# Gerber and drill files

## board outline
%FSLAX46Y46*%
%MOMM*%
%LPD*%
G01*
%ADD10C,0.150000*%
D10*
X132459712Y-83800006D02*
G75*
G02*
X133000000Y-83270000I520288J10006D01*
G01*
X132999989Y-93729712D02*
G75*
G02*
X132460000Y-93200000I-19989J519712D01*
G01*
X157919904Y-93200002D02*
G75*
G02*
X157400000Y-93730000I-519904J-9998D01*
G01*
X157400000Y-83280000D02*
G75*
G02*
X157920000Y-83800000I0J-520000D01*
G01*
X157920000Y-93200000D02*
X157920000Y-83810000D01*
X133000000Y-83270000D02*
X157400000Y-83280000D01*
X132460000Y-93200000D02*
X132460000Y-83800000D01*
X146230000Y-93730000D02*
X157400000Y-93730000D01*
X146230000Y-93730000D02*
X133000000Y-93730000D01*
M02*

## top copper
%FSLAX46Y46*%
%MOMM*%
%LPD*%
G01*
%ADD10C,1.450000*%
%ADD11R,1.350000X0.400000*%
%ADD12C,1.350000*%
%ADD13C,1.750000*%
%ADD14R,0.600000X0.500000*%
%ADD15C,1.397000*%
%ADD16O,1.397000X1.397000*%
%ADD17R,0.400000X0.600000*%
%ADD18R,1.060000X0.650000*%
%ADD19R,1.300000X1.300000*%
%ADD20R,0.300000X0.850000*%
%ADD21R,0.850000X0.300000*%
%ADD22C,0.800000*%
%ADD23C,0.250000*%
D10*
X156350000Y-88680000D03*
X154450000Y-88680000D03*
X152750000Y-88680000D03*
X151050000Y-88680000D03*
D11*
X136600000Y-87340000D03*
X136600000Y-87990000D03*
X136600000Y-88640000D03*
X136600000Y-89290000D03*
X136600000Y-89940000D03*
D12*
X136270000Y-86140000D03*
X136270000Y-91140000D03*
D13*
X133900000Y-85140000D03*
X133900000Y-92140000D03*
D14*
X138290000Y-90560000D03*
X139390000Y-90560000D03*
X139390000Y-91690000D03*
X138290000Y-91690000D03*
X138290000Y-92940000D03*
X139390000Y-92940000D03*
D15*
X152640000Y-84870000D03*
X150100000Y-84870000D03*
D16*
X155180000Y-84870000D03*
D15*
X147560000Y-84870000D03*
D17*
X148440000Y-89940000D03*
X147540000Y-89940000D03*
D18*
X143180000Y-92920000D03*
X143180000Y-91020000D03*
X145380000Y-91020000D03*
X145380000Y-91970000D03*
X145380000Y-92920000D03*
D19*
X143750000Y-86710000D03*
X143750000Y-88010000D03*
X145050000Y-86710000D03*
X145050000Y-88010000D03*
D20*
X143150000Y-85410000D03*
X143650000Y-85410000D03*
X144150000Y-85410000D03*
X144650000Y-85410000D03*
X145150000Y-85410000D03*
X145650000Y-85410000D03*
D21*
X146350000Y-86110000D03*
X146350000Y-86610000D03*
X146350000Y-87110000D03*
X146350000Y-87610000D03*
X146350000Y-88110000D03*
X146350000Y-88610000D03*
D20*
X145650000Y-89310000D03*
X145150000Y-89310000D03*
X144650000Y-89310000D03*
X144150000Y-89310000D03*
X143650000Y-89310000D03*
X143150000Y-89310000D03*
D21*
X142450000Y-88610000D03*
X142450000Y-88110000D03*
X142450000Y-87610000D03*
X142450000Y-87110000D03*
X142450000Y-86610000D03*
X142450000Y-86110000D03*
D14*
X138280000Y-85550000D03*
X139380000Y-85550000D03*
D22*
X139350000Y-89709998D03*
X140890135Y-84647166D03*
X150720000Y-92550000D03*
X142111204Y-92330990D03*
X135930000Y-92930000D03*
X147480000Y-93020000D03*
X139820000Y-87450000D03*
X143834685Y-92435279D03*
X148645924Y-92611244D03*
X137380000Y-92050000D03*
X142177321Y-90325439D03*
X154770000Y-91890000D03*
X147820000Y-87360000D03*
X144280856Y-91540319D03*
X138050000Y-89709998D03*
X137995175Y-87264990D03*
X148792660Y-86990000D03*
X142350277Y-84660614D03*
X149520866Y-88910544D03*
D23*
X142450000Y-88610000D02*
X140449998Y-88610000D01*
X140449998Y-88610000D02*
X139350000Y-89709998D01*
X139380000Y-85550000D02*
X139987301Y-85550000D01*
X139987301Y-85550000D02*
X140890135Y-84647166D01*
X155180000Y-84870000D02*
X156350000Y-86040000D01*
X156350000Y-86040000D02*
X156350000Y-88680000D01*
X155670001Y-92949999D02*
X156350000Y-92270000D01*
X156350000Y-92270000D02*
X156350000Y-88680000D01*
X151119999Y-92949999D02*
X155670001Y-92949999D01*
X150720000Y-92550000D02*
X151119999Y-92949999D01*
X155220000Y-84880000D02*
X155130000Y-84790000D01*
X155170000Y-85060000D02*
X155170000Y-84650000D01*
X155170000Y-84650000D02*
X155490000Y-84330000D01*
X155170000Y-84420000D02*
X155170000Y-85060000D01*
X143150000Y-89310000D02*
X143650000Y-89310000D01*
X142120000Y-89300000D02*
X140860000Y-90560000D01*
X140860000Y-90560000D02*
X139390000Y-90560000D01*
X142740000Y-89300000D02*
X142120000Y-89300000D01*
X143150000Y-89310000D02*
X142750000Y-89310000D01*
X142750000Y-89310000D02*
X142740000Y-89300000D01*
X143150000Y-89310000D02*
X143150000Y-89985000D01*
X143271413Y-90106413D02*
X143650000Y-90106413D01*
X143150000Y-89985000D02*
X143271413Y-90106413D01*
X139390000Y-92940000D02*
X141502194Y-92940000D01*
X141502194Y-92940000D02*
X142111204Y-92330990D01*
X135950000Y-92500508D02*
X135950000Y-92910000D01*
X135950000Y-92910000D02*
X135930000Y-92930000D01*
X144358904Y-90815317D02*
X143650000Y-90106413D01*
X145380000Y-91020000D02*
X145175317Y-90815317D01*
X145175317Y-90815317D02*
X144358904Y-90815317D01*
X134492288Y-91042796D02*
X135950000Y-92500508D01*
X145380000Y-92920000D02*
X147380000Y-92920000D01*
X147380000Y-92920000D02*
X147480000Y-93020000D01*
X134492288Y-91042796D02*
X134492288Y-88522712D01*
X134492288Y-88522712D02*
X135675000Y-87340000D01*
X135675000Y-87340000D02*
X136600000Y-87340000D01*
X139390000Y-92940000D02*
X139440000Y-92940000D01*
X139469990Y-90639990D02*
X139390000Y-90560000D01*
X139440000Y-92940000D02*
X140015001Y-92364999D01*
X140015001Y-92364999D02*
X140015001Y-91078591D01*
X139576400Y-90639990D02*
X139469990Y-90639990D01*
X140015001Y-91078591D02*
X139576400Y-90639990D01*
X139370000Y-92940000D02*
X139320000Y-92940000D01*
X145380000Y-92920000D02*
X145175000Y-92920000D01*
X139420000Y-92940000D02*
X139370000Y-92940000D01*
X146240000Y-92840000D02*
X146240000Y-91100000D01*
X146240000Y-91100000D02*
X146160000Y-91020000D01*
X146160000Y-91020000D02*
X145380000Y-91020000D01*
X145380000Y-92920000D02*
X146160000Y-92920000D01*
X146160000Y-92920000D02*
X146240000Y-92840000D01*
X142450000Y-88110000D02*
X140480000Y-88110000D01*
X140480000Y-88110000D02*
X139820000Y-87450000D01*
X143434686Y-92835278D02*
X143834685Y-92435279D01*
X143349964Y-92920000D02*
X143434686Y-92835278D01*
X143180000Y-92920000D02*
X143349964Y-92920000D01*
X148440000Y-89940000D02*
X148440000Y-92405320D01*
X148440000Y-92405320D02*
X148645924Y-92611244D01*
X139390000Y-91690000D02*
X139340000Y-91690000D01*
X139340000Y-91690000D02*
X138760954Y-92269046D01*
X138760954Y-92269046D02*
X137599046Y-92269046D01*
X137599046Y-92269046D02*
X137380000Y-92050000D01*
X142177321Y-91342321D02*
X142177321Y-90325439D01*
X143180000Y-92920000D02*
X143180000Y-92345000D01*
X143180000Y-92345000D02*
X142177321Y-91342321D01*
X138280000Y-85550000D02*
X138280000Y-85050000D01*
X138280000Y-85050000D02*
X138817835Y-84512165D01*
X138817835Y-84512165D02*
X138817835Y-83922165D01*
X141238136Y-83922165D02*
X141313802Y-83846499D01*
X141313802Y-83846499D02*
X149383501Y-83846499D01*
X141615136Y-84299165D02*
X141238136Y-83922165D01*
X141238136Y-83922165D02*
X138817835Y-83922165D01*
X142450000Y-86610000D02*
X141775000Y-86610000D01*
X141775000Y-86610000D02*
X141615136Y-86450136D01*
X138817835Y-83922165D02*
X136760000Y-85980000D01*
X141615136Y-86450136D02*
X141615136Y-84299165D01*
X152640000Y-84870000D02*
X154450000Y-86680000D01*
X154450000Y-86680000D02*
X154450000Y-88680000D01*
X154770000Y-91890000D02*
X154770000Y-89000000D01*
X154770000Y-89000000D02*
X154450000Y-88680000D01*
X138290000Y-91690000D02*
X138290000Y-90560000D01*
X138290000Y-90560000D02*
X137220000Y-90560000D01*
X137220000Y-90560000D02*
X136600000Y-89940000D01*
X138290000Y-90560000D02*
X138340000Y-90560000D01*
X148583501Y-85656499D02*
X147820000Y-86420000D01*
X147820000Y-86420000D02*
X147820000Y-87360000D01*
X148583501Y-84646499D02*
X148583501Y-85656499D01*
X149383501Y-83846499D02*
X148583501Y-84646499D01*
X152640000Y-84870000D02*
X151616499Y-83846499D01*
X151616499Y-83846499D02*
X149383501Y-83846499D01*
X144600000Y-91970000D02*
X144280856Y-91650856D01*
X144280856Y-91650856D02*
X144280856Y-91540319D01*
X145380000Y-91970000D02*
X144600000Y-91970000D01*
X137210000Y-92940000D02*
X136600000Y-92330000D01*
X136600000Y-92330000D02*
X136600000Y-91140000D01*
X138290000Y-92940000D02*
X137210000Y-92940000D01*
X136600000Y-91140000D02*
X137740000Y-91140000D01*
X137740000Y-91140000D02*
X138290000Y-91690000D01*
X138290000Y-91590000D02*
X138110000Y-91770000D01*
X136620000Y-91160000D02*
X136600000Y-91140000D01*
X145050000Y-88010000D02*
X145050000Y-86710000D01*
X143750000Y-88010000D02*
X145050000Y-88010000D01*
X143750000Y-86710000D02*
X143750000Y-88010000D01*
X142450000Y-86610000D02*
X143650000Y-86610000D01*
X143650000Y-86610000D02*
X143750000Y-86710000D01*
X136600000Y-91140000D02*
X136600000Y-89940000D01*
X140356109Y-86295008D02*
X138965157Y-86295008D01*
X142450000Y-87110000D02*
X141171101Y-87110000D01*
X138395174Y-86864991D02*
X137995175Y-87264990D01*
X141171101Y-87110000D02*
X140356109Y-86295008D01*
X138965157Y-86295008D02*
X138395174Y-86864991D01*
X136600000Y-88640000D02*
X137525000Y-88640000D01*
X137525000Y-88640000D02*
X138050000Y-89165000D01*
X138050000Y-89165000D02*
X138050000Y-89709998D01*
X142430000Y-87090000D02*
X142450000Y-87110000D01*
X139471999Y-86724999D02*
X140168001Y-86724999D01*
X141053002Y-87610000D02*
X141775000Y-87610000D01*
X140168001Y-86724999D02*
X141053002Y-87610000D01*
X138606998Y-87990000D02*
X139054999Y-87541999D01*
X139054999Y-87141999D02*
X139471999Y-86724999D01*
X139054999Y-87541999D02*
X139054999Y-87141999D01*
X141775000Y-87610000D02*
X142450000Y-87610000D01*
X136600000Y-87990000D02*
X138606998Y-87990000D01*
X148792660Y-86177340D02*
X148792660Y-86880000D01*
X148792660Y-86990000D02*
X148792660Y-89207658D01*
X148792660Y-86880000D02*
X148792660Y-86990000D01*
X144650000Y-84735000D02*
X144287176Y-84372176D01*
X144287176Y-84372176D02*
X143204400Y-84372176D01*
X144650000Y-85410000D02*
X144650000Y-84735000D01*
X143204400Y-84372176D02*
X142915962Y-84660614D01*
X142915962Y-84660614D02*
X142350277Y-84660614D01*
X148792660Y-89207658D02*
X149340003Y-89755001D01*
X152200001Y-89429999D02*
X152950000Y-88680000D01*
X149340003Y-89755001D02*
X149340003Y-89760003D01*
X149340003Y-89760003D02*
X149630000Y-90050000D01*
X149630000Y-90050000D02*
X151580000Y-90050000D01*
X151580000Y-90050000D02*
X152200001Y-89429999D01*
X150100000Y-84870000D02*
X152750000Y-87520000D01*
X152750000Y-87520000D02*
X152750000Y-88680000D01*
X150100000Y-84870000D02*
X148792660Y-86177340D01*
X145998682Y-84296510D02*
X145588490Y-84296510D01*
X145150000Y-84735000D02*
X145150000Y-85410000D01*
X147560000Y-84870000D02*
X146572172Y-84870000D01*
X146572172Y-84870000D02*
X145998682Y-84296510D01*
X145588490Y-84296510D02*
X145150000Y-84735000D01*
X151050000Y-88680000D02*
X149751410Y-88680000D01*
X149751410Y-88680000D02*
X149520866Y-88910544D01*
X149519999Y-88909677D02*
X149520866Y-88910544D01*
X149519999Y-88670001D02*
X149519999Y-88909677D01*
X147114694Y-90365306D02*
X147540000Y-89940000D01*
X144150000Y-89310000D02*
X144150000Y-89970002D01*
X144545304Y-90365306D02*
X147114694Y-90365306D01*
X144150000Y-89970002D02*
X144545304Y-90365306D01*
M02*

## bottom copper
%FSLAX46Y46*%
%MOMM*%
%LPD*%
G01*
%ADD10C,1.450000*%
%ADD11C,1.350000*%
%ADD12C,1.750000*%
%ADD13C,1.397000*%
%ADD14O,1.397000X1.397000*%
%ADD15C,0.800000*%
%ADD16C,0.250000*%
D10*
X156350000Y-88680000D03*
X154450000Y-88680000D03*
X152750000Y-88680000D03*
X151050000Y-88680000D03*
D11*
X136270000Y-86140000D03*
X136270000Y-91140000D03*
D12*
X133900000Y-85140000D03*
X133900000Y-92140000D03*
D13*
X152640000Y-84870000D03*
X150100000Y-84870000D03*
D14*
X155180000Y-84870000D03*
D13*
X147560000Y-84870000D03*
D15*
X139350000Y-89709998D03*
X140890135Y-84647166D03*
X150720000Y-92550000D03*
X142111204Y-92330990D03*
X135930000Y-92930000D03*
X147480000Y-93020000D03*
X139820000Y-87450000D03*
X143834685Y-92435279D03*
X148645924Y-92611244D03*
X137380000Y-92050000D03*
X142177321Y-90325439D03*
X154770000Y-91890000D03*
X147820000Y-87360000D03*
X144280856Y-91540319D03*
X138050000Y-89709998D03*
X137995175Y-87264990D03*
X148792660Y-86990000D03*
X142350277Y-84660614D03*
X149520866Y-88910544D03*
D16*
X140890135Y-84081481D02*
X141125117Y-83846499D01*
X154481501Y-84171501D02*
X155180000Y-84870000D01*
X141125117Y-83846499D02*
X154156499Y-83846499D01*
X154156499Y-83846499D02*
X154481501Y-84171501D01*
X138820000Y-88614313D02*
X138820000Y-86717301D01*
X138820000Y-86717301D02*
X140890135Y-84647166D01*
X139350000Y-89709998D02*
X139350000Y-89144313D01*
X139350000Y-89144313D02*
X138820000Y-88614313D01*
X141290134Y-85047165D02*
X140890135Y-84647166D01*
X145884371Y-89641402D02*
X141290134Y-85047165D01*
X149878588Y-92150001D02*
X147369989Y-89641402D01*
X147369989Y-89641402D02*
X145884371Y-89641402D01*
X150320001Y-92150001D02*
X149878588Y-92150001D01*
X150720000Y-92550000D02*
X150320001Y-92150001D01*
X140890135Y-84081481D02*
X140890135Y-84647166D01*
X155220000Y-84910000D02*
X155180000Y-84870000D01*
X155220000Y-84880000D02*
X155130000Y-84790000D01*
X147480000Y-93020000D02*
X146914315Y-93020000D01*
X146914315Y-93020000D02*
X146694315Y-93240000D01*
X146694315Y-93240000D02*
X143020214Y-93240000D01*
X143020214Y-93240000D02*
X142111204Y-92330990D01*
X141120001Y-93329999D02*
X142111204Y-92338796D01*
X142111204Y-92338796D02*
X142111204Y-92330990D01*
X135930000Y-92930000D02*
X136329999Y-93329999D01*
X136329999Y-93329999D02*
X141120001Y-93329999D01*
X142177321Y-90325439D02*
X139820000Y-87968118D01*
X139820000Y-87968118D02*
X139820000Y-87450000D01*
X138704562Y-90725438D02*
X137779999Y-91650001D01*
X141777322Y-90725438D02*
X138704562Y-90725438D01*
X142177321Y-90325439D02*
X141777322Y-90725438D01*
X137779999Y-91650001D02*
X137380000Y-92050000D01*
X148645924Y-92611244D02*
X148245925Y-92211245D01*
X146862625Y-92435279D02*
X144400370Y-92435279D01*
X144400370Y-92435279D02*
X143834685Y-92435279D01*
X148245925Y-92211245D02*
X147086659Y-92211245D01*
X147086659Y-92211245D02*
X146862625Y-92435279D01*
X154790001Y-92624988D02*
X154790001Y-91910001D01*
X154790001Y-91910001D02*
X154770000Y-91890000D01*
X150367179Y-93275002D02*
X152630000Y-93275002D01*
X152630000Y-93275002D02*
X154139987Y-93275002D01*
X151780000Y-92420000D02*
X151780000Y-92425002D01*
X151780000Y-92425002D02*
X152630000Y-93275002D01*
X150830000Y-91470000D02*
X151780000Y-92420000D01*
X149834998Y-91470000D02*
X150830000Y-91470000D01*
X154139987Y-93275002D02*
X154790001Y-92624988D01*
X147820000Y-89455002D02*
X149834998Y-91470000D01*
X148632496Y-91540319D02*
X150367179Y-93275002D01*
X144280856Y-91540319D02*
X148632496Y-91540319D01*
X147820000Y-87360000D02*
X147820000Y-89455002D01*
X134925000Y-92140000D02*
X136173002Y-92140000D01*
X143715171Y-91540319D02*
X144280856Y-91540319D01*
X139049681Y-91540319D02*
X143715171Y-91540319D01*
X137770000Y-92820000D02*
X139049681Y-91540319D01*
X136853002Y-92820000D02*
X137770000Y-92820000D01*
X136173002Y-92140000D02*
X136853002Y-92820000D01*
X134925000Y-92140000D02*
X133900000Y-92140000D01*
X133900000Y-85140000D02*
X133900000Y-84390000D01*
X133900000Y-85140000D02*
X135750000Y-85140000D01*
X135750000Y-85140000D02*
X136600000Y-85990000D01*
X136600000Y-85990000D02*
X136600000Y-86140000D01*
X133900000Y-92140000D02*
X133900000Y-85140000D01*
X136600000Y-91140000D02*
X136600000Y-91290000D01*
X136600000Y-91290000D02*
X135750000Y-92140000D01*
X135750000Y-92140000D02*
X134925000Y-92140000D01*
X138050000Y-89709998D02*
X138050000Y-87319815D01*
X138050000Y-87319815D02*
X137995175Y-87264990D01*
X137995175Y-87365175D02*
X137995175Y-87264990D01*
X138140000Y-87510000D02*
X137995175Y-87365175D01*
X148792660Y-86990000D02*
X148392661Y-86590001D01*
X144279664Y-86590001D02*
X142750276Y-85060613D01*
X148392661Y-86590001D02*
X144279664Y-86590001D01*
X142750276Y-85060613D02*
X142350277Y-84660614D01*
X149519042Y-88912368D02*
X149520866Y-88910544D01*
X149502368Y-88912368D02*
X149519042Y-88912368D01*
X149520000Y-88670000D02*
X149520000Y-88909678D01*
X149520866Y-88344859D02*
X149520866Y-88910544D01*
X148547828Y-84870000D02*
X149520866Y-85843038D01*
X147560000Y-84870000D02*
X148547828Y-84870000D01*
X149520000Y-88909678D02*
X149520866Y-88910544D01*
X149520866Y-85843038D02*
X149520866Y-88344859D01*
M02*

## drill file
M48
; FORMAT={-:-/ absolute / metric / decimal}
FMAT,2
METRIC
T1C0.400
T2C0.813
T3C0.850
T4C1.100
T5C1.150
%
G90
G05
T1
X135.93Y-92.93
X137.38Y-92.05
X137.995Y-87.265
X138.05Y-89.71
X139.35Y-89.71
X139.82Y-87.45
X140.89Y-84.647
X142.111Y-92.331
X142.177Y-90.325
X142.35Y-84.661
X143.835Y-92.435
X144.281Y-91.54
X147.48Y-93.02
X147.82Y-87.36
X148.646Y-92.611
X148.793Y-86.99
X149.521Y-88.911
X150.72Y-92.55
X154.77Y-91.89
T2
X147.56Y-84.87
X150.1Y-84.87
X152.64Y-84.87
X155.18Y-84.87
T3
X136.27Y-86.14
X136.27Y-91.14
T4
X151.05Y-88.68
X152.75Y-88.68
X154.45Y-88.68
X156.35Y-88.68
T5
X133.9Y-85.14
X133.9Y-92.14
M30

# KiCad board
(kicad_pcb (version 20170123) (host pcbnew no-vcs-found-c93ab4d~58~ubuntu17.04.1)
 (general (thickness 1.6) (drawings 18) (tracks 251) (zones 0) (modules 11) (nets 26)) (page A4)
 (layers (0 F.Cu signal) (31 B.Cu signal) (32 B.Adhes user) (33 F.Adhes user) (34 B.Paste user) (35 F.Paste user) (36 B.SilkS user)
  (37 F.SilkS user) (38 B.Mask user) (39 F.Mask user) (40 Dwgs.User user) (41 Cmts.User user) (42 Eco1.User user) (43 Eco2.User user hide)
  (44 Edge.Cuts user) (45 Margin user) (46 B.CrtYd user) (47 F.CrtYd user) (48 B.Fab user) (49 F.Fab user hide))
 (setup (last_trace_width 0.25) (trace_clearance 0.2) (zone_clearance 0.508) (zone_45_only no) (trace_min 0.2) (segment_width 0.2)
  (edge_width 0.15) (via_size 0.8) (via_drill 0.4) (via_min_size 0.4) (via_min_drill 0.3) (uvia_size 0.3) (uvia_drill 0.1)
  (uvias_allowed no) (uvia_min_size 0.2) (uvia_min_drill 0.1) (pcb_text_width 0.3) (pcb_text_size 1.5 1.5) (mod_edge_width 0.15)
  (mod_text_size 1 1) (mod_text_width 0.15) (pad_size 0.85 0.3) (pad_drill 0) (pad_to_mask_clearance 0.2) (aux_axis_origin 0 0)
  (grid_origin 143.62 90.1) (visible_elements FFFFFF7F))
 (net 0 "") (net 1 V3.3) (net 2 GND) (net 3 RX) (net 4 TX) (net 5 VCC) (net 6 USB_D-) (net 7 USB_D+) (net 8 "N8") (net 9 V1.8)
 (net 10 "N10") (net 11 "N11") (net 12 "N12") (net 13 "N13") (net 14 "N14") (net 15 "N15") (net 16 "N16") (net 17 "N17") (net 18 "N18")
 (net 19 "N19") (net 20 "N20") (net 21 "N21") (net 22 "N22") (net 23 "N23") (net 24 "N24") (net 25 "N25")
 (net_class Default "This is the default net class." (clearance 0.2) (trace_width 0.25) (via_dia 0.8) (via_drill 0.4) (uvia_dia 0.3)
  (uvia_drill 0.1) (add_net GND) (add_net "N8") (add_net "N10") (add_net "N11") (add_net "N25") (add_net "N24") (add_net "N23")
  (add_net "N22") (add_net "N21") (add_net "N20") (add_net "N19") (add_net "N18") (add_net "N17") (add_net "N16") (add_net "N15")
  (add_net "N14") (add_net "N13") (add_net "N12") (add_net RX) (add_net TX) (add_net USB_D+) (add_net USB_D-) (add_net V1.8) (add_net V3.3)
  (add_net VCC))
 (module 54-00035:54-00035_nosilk (layer F.Cu) (at 149.1 88.68)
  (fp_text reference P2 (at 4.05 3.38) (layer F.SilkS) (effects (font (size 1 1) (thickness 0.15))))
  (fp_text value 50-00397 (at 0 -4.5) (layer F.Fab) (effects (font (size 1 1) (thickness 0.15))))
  (pad 4 thru_hole circle (at 7.25 0) (size 1.45 1.45) (drill 1.1) (layers *.Cu *.Mask) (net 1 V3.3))
  (pad 3 thru_hole circle (at 5.35 0) (size 1.45 1.45) (drill 1.1) (layers *.Cu *.Mask) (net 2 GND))
  (pad 2 thru_hole circle (at 3.65 0) (size 1.45 1.45) (drill 1.1) (layers *.Cu *.Mask) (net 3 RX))
  (pad 1 thru_hole circle (at 1.95 0) (size 1.45 1.45) (drill 1.1) (layers *.Cu *.Mask) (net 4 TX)))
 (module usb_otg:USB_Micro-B (layer F.Cu) (at 135.25 88.64 270)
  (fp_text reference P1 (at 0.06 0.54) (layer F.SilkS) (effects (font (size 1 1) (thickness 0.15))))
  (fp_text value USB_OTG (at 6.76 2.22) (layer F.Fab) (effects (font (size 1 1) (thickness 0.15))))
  (pad 1 smd rect (at -1.3 -1.35) (size 1.35 0.4) (layers F.Cu F.Paste F.Mask) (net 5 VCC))
  (pad 2 smd rect (at -0.65 -1.35) (size 1.35 0.4) (layers F.Cu F.Paste F.Mask) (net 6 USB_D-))
  (pad 3 smd rect (at 0 -1.35) (size 1.35 0.4) (layers F.Cu F.Paste F.Mask) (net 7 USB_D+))
  (pad 4 smd rect (at 0.65 -1.35) (size 1.35 0.4) (layers F.Cu F.Paste F.Mask) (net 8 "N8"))
  (pad 5 smd rect (at 1.3 -1.35) (size 1.35 0.4) (layers F.Cu F.Paste F.Mask) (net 2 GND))
  (pad 6 thru_hole circle (at -2.5 -1.02) (size 1.35 1.35) (drill 0.85) (layers *.Cu *.Mask) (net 2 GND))
  (pad 6 thru_hole circle (at 2.5 -1.02) (size 1.35 1.35) (drill 0.85) (layers *.Cu *.Mask) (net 2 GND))
  (pad 6 thru_hole circle (at -3.5 1.35) (size 1.75 1.75) (drill 1.15) (layers *.Cu *.Mask) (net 2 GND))
  (pad 6 thru_hole circle (at 3.5 1.35) (size 1.75 1.75) (drill 1.15) (layers *.Cu *.Mask) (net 2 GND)))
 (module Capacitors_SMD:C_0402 (layer F.Cu) (at 138.84 90.56)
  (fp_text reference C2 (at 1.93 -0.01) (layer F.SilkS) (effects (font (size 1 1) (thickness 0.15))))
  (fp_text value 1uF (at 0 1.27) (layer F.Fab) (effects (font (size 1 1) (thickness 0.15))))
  (pad 1 smd rect (at -0.55 0) (size 0.6 0.5) (layers F.Cu F.Paste F.Mask) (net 2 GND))
  (pad 2 smd rect (at 0.55 0) (size 0.6 0.5) (layers F.Cu F.Paste F.Mask) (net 5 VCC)))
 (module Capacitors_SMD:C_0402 (layer F.Cu) (at 138.84 91.69 180)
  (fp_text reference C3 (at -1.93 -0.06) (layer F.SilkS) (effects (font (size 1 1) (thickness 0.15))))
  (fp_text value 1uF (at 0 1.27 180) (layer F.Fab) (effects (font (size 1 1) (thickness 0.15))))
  (pad 1 smd rect (at -0.55 0 180) (size 0.6 0.5) (layers F.Cu F.Paste F.Mask) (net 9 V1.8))
  (pad 2 smd rect (at 0.55 0 180) (size 0.6 0.5) (layers F.Cu F.Paste F.Mask) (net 2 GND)))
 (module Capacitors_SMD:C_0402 (layer F.Cu) (at 138.84 92.94 180)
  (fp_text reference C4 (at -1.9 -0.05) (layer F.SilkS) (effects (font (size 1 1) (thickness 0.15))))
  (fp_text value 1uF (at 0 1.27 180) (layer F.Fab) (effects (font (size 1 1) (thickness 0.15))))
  (pad 2 smd rect (at 0.55 0 180) (size 0.6 0.5) (layers F.Cu F.Paste F.Mask) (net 2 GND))
  (pad 1 smd rect (at -0.55 0 180) (size 0.6 0.5) (layers F.Cu F.Paste F.Mask) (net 5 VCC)))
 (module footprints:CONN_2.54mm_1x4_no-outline (layer F.Cu) (at 151.37 84.87)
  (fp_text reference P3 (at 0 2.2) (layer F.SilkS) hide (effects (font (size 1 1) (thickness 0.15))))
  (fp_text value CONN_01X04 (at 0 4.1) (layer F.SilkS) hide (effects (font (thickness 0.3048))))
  (pad 2 thru_hole circle (at 1.27 0) (size 1.397 1.397) (drill 0.8128) (layers *.Cu *.Mask F.SilkS) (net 2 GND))
  (pad 3 thru_hole circle (at -1.27 0) (size 1.397 1.397) (drill 0.8128) (layers *.Cu *.Mask F.SilkS) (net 3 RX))
  (pad 1 thru_hole oval (at 3.81 0) (size 1.397 1.397) (drill 0.8128) (layers *.Cu *.Mask F.SilkS) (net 1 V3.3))
  (pad 4 thru_hole circle (at -3.81 0) (size 1.397 1.397) (drill 0.8128) (layers *.Cu *.Mask F.SilkS) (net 4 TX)))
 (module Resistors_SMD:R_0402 (layer F.Cu) (at 147.99 89.94)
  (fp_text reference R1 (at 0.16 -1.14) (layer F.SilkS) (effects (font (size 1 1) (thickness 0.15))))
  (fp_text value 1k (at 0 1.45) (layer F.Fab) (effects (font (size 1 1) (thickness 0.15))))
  (pad 2 smd rect (at 0.45 0) (size 0.4 0.6) (layers F.Cu F.Paste F.Mask) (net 9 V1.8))
  (pad 1 smd rect (at -0.45 0) (size 0.4 0.6) (layers F.Cu F.Paste F.Mask) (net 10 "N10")))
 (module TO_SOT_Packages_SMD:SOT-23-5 (layer F.Cu) (at 144.28 91.97 180)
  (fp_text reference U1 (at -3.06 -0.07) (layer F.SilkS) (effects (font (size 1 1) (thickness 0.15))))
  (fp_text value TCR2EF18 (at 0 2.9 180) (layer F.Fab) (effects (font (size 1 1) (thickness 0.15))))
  (pad 5 smd rect (at 1.1 -0.95 180) (size 1.06 0.65) (layers F.Cu F.Paste F.Mask) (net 9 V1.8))
  (pad 4 smd rect (at 1.1 0.95 180) (size 1.06 0.65) (layers F.Cu F.Paste F.Mask) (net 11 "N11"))
  (pad 3 smd rect (at -1.1 0.95 180) (size 1.06 0.65) (layers F.Cu F.Paste F.Mask) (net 5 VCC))
  (pad 2 smd rect (at -1.1 0 180) (size 1.06 0.65) (layers F.Cu F.Paste F.Mask) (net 2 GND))
  (pad 1 smd rect (at -1.1 -0.95 180) (size 1.06 0.65) (layers F.Cu F.Paste F.Mask) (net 5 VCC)))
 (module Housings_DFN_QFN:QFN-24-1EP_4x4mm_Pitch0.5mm (layer F.Cu) (at 144.4 87.36)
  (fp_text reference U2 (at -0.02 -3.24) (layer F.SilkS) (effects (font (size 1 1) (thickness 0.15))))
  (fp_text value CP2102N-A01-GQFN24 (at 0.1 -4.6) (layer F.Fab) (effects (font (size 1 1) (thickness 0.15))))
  (pad 25 smd rect (at -0.65 -0.65) (size 1.3 1.3) (layers F.Cu F.Paste F.Mask) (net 2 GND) (solder_paste_margin_ratio -0.2))
  (pad 25 smd rect (at -0.65 0.65) (size 1.3 1.3) (layers F.Cu F.Paste F.Mask) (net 2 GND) (solder_paste_margin_ratio -0.2))
  (pad 25 smd rect (at 0.65 -0.65) (size 1.3 1.3) (layers F.Cu F.Paste F.Mask) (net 2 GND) (solder_paste_margin_ratio -0.2))
  (pad 25 smd rect (at 0.65 0.65) (size 1.3 1.3) (layers F.Cu F.Paste F.Mask) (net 2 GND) (solder_paste_margin_ratio -0.2))
  (pad 24 smd rect (at -1.25 -1.95 90) (size 0.85 0.3) (layers F.Cu F.Paste F.Mask) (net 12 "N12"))
  (pad 23 smd rect (at -0.75 -1.95 90) (size 0.85 0.3) (layers F.Cu F.Paste F.Mask) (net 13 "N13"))
  (pad 22 smd rect (at -0.25 -1.95 90) (size 0.85 0.3) (layers F.Cu F.Paste F.Mask) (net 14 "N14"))
  (pad 21 smd rect (at 0.25 -1.95 90) (size 0.85 0.3) (layers F.Cu F.Paste F.Mask) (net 3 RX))
  (pad 20 smd rect (at 0.75 -1.95 90) (size 0.85 0.3) (layers F.Cu F.Paste F.Mask) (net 4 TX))
  (pad 19 smd rect (at 1.25 -1.95 90) (size 0.85 0.3) (layers F.Cu F.Paste F.Mask) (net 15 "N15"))
  (pad 18 smd rect (at 1.95 -1.25) (size 0.85 0.3) (layers F.Cu F.Paste F.Mask) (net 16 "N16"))
  (pad 17 smd rect (at 1.95 -0.75) (size 0.85 0.3) (layers F.Cu F.Paste F.Mask) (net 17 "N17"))
  (pad 16 smd rect (at 1.95 -0.25) (size 0.85 0.3) (layers F.Cu F.Paste F.Mask) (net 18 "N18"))
  (pad 15 smd rect (at 1.95 0.25) (size 0.85 0.3) (layers F.Cu F.Paste F.Mask) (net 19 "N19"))
  (pad 14 smd rect (at 1.95 0.75) (size 0.85 0.3) (layers F.Cu F.Paste F.Mask) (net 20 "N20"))
  (pad 13 smd rect (at 1.95 1.25) (size 0.85 0.3) (layers F.Cu F.Paste F.Mask) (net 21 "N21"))
  (pad 12 smd rect (at 1.25 1.95 90) (size 0.85 0.3) (layers F.Cu F.Paste F.Mask) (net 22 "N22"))
  (pad 11 smd rect (at 0.75 1.95 90) (size 0.85 0.3) (layers F.Cu F.Paste F.Mask) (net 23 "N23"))
  (pad 10 smd rect (at 0.25 1.95 90) (size 0.85 0.3) (layers F.Cu F.Paste F.Mask) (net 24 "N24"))
  (pad 9 smd rect (at -0.25 1.95 90) (size 0.85 0.3) (layers F.Cu F.Paste F.Mask) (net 10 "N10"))
  (pad 8 smd rect (at -0.75 1.95 90) (size 0.85 0.3) (layers F.Cu F.Paste F.Mask) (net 5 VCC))
  (pad 7 smd rect (at -1.25 1.95 90) (size 0.85 0.3) (layers F.Cu F.Paste F.Mask) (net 5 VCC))
  (pad 6 smd rect (at -1.95 1.25) (size 0.85 0.3) (layers F.Cu F.Paste F.Mask) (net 1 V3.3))
  (pad 5 smd rect (at -1.95 0.75) (size 0.85 0.3) (layers F.Cu F.Paste F.Mask) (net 9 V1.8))
  (pad 4 smd rect (at -1.95 0.25) (size 0.85 0.3) (layers F.Cu F.Paste F.Mask) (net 6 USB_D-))
  (pad 3 smd rect (at -1.95 -0.25) (size 0.85 0.3) (layers F.Cu F.Paste F.Mask) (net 7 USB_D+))
  (pad 2 smd rect (at -1.95 -0.75) (size 0.85 0.3) (layers F.Cu F.Paste F.Mask) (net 2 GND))
  (pad 1 smd rect (at -1.95 -1.25) (size 0.85 0.3) (layers F.Cu F.Paste F.Mask) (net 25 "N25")))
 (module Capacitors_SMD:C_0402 (layer F.Cu) (at 138.83 85.55 180)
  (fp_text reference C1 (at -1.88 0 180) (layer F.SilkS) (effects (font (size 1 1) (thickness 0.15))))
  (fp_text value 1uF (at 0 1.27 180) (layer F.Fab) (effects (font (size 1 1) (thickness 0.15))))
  (pad 2 smd rect (at 0.55 0 180) (size 0.6 0.5) (layers F.Cu F.Paste F.Mask) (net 2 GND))
  (pad 1 smd rect (at -0.55 0 180) (size 0.6 0.5) (layers F.Cu F.Paste F.Mask) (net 1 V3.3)))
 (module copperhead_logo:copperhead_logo (layer B.Cu) (at 141.43 88.4)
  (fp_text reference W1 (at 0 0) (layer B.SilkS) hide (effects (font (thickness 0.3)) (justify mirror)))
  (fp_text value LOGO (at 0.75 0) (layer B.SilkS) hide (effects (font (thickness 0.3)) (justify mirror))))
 (gr_arc (start 132.98 83.79) (end 133 83.27) (angle -93.30435508) (layer Edge.Cuts) (width 0.15))
 (gr_arc (start 132.98 93.21) (end 132.46 93.2) (angle -93.30431274) (layer Edge.Cuts) (width 0.15))
 (gr_arc (start 157.4 93.21) (end 157.4 93.73) (angle -91.10169129) (layer Edge.Cuts) (width 0.15))
 (gr_arc (start 157.4 83.8) (end 157.92 83.8) (angle -90) (layer Edge.Cuts) (width 0.15))
 (gr_line (start 157.92 93.2) (end 157.92 83.81) (layer Edge.Cuts) (width 0.15))
 (gr_line (start 133 83.27) (end 157.4 83.28) (layer Edge.Cuts) (width 0.15))
 (gr_line (start 132.46 93.2) (end 132.46 83.8) (layer Edge.Cuts) (width 0.15))
 (gr_line (start 146.23 93.73) (end 157.4 93.73) (layer Edge.Cuts) (width 0.15))
 (gr_line (start 146.23 93.73) (end 133 93.73) (layer Edge.Cuts) (width 0.15))
 (segment (start 140.890135 84.081481) (end 141.125117 83.846499) (width 0.25) (layer B.Cu) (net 1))
 (segment (start 154.481501 84.171501) (end 155.18 84.87) (width 0.25) (layer B.Cu) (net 1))
 (segment (start 141.125117 83.846499) (end 154.156499 83.846499) (width 0.25) (layer B.Cu) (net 1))
 (segment (start 154.156499 83.846499) (end 154.481501 84.171501) (width 0.25) (layer B.Cu) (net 1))
 (segment (start 138.82 88.614313) (end 138.82 86.717301) (width 0.25) (layer B.Cu) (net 1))
 (segment (start 138.82 86.717301) (end 140.890135 84.647166) (width 0.25) (layer B.Cu) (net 1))
 (segment (start 139.35 89.709998) (end 139.35 89.144313) (width 0.25) (layer B.Cu) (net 1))
 (segment (start 139.35 89.144313) (end 138.82 88.614313) (width 0.25) (layer B.Cu) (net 1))
 (segment (start 142.45 88.61) (end 140.449998 88.61) (width 0.25) (layer F.Cu) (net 1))
 (segment (start 140.449998 88.61) (end 139.35 89.709998) (width 0.25) (layer F.Cu) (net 1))
 (segment (start 139.38 85.55) (end 139.987301 85.55) (width 0.25) (layer F.Cu) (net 1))
 (segment (start 139.987301 85.55) (end 140.890135 84.647166) (width 0.25) (layer F.Cu) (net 1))
 (segment (start 155.18 84.87) (end 156.35 86.04) (width 0.25) (layer F.Cu) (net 1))
 (segment (start 156.35 86.04) (end 156.35 88.68) (width 0.25) (layer F.Cu) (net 1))
 (segment (start 155.670001 92.949999) (end 156.35 92.27) (width 0.25) (layer F.Cu) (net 1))
 (segment (start 156.35 92.27) (end 156.35 88.68) (width 0.25) (layer F.Cu) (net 1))
 (segment (start 151.119999 92.949999) (end 155.670001 92.949999) (width 0.25) (layer F.Cu) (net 1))
 (segment (start 150.72 92.55) (end 151.119999 92.949999) (width 0.25) (layer F.Cu) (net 1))
 (segment (start 141.290134 85.047165) (end 140.890135 84.647166) (width 0.25) (layer B.Cu) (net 1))
 (segment (start 145.884371 89.641402) (end 141.290134 85.047165) (width 0.25) (layer B.Cu) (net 1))
 (segment (start 149.878588 92.150001) (end 147.369989 89.641402) (width 0.25) (layer B.Cu) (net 1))
 (segment (start 147.369989 89.641402) (end 145.884371 89.641402) (width 0.25) (layer B.Cu) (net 1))
 (segment (start 150.320001 92.150001) (end 149.878588 92.150001) (width 0.25) (layer B.Cu) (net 1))
 (segment (start 150.72 92.55) (end 150.320001 92.150001) (width 0.25) (layer B.Cu) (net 1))
 (segment (start 140.890135 84.081481) (end 140.890135 84.647166) (width 0.25) (layer B.Cu) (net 1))
 (segment (start 155.22 84.91) (end 155.18 84.87) (width 0.25) (layer B.Cu) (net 1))
 (segment (start 155.22 84.88) (end 155.13 84.79) (width 0.25) (layer B.Cu) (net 1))
 (segment (start 155.22 84.88) (end 155.13 84.79) (width 0.25) (layer F.Cu) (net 1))
 (segment (start 155.17 85.06) (end 155.17 84.65) (width 0.25) (layer F.Cu) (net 1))
 (segment (start 155.17 84.65) (end 155.49 84.33) (width 0.25) (layer F.Cu) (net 1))
 (segment (start 155.17 84.42) (end 155.17 85.06) (width 0.25) (layer F.Cu) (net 1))
 (segment (start 143.15 89.31) (end 143.65 89.31) (width 0.25) (layer F.Cu) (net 5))
 (segment (start 142.12 89.3) (end 140.86 90.56) (width 0.25) (layer F.Cu) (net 5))
 (segment (start 140.86 90.56) (end 139.39 90.56) (width 0.25) (layer F.Cu) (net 5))
 (segment (start 142.74 89.3) (end 142.12 89.3) (width 0.25) (layer F.Cu) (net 5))
 (segment (start 143.15 89.31) (end 142.75 89.31) (width 0.25) (layer F.Cu) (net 5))
 (segment (start 142.75 89.31) (end 142.74 89.3) (width 0.25) (layer F.Cu) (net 5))
 (segment (start 143.15 89.31) (end 143.15 89.985) (width 0.25) (layer F.Cu) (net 5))
 (segment (start 143.271413 90.106413) (end 143.65 90.106413) (width 0.25) (layer F.Cu) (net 5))
 (segment (start 143.15 89.985) (end 143.271413 90.106413) (width 0.25) (layer F.Cu) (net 5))
 (segment (start 139.39 92.94) (end 141.502194 92.94) (width 0.25) (layer F.Cu) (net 5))
 (segment (start 141.502194 92.94) (end 142.111204 92.33099) (width 0.25) (layer F.Cu) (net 5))
 (segment (start 147.48 93.02) (end 146.914315 93.02) (width 0.25) (layer B.Cu) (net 5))
 (segment (start 146.914315 93.02) (end 146.694315 93.24) (width 0.25) (layer B.Cu) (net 5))
 (segment (start 146.694315 93.24) (end 143.020214 93.24) (width 0.25) (layer B.Cu) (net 5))
 (segment (start 143.020214 93.24) (end 142.111204 92.33099) (width 0.25) (layer B.Cu) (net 5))
 (segment (start 141.120001 93.329999) (end 142.111204 92.338796) (width 0.25) (layer B.Cu) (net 5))
 (segment (start 142.111204 92.338796) (end 142.111204 92.33099) (width 0.25) (layer B.Cu) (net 5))
 (segment (start 135.93 92.93) (end 136.329999 93.329999) (width 0.25) (layer B.Cu) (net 5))
 (segment (start 136.329999 93.329999) (end 141.120001 93.329999) (width 0.25) (layer B.Cu) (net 5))
 (segment (start 135.95 92.500508) (end 135.95 92.91) (width 0.25) (layer F.Cu) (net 5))
 (segment (start 135.95 92.91) (end 135.93 92.93) (width 0.25) (layer F.Cu) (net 5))
 (segment (start 144.358904 90.815317) (end 143.65 90.106413) (width 0.25) (layer F.Cu) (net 5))
 (segment (start 145.38 91.02) (end 145.175317 90.815317) (width 0.25) (layer F.Cu) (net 5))
 (segment (start 145.175317 90.815317) (end 144.358904 90.815317) (width 0.25) (layer F.Cu) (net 5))
 (segment (start 134.492288 91.042796) (end 135.95 92.500508) (width 0.25) (layer F.Cu) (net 5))
 (segment (start 145.38 92.92) (end 147.38 92.92) (width 0.25) (layer F.Cu) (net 5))
 (segment (start 147.38 92.92) (end 147.48 93.02) (width 0.25) (layer F.Cu) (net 5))
 (segment (start 134.492288 91.042796) (end 134.492288 88.522712) (width 0.25) (layer F.Cu) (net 5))
 (segment (start 134.492288 88.522712) (end 135.675 87.34) (width 0.25) (layer F.Cu) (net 5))
 (segment (start 135.675 87.34) (end 136.6 87.34) (width 0.25) (layer F.Cu) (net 5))
 (segment (start 139.39 92.94) (end 139.44 92.94) (width 0.25) (layer F.Cu) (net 5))
 (segment (start 139.46999 90.63999) (end 139.39 90.56) (width 0.25) (layer F.Cu) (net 5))
 (segment (start 139.44 92.94) (end 140.015001 92.364999) (width 0.25) (layer F.Cu) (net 5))
 (segment (start 140.015001 92.364999) (end 140.015001 91.078591) (width 0.25) (layer F.Cu) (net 5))
 (segment (start 139.5764 90.63999) (end 139.46999 90.63999) (width 0.25) (layer F.Cu) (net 5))
 (segment (start 140.015001 91.078591) (end 139.5764 90.63999) (width 0.25) (layer F.Cu) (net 5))
 (segment (start 139.37 92.94) (end 139.32 92.94) (width 0.25) (layer F.Cu) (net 5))
 (segment (start 145.38 92.92) (end 145.175 92.92) (width 0.25) (layer F.Cu) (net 5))
 (segment (start 139.42 92.94) (end 139.37 92.94) (width 0.25) (layer F.Cu) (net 5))
 (segment (start 146.24 92.84) (end 146.24 91.1) (width 0.25) (layer F.Cu) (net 5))
 (segment (start 146.24 91.1) (end 146.16 91.02) (width 0.25) (layer F.Cu) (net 5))
 (segment (start 146.16 91.02) (end 145.38 91.02) (width 0.25) (layer F.Cu) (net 5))
 (segment (start 145.38 92.92) (end 146.16 92.92) (width 0.25) (layer F.Cu) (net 5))
 (segment (start 146.16 92.92) (end 146.24 92.84) (width 0.25) (layer F.Cu) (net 5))
 (segment (start 142.177321 90.325439) (end 139.82 87.968118) (width 0.25) (layer B.Cu) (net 9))
 (segment (start 139.82 87.968118) (end 139.82 87.45) (width 0.25) (layer B.Cu) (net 9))
 (segment (start 142.45 88.11) (end 140.48 88.11) (width 0.25) (layer F.Cu) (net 9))
 (segment (start 140.48 88.11) (end 139.82 87.45) (width 0.25) (layer F.Cu) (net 9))
 (segment (start 138.704562 90.725438) (end 137.779999 91.650001) (width 0.25) (layer B.Cu) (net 9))
 (segment (start 141.777322 90.725438) (end 138.704562 90.725438) (width 0.25) (layer B.Cu) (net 9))
 (segment (start 142.177321 90.325439) (end 141.777322 90.725438) (width 0.25) (layer B.Cu) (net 9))
 (segment (start 137.779999 91.650001) (end 137.38 92.05) (width 0.25) (layer B.Cu) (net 9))
 (segment (start 148.645924 92.611244) (end 148.245925 92.211245) (width 0.25) (layer B.Cu) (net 9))
 (segment (start 143.434686 92.835278) (end 143.834685 92.435279) (width 0.25) (layer F.Cu) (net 9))
 (segment (start 143.349964 92.92) (end 143.434686 92.835278) (width 0.25) (layer F.Cu) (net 9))
 (segment (start 146.862625 92.435279) (end 144.40037 92.435279) (width 0.25) (layer B.Cu) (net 9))
 (segment (start 143.18 92.92) (end 143.349964 92.92) (width 0.25) (layer F.Cu) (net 9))
 (segment (start 144.40037 92.435279) (end 143.834685 92.435279) (width 0.25) (layer B.Cu) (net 9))
 (segment (start 148.245925 92.211245) (end 147.086659 92.211245) (width 0.25) (layer B.Cu) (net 9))
 (segment (start 147.086659 92.211245) (end 146.862625 92.435279) (width 0.25) (layer B.Cu) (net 9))
 (segment (start 148.44 89.94) (end 148.44 92.40532) (width 0.25) (layer F.Cu) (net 9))
 (segment (start 148.44 92.40532) (end 148.645924 92.611244) (width 0.25) (layer F.Cu) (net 9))
 (segment (start 139.39 91.69) (end 139.34 91.69) (width 0.25) (layer F.Cu) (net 9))
 (segment (start 139.34 91.69) (end 138.760954 92.269046) (width 0.25) (layer F.Cu) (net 9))
 (segment (start 138.760954 92.269046) (end 137.599046 92.269046) (width 0.25) (layer F.Cu) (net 9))
 (segment (start 137.599046 92.269046) (end 137.38 92.05) (width 0.25) (layer F.Cu) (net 9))
 (segment (start 142.177321 91.342321) (end 142.177321 90.325439) (width 0.25) (layer F.Cu) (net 9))
 (segment (start 143.18 92.92) (end 143.18 92.345) (width 0.25) (layer F.Cu) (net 9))
 (segment (start 143.18 92.345) (end 142.177321 91.342321) (width 0.25) (layer F.Cu) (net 9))
 (segment (start 138.28 85.55) (end 138.28 85.05) (width 0.25) (layer F.Cu) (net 2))
 (segment (start 138.28 85.05) (end 138.817835 84.512165) (width 0.25) (layer F.Cu) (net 2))
 (segment (start 138.817835 84.512165) (end 138.817835 83.922165) (width 0.25) (layer F.Cu) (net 2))
 (segment (start 141.238136 83.922165) (end 141.313802 83.846499) (width 0.25) (layer F.Cu) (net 2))
 (segment (start 141.313802 83.846499) (end 149.383501 83.846499) (width 0.25) (layer F.Cu) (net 2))
 (segment (start 141.615136 84.299165) (end 141.238136 83.922165) (width 0.25) (layer F.Cu) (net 2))
 (segment (start 141.238136 83.922165) (end 138.817835 83.922165) (width 0.25) (layer F.Cu) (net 2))
 (segment (start 142.45 86.61) (end 141.775 86.61) (width 0.25) (layer F.Cu) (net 2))
 (segment (start 141.775 86.61) (end 141.615136 86.450136) (width 0.25) (layer F.Cu) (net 2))
 (segment (start 138.817835 83.922165) (end 136.76 85.98) (width 0.25) (layer F.Cu) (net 2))
 (segment (start 141.615136 86.450136) (end 141.615136 84.299165) (width 0.25) (layer F.Cu) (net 2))
 (segment (start 152.64 84.87) (end 154.45 86.68) (width 0.25) (layer F.Cu) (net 2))
 (segment (start 154.45 86.68) (end 154.45 88.68) (width 0.25) (layer F.Cu) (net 2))
 (segment (start 154.77 91.89) (end 154.77 89) (width 0.25) (layer F.Cu) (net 2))
 (segment (start 154.77 89) (end 154.45 88.68) (width 0.25) (layer F.Cu) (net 2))
 (segment (start 154.790001 92.624988) (end 154.790001 91.910001) (width 0.25) (layer B.Cu) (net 2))
 (segment (start 154.790001 91.910001) (end 154.77 91.89) (width 0.25) (layer B.Cu) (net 2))
 (segment (start 138.29 91.69) (end 138.29 90.56) (width 0.25) (layer F.Cu) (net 2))
 (segment (start 138.29 90.56) (end 137.22 90.56) (width 0.25) (layer F.Cu) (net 2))
 (segment (start 137.22 90.56) (end 136.6 89.94) (width 0.25) (layer F.Cu) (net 2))
 (segment (start 138.29 90.56) (end 138.34 90.56) (width 0.25) (layer F.Cu) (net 2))
 (segment (start 150.367179 93.275002) (end 152.63 93.275002) (width 0.25) (layer B.Cu) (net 2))
 (segment (start 152.63 93.275002) (end 154.139987 93.275002) (width 0.25) (layer B.Cu) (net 2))
 (segment (start 151.78 92.42) (end 151.78 92.425002) (width 0.25) (layer B.Cu) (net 2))
 (segment (start 151.78 92.425002) (end 152.63 93.275002) (width 0.25) (layer B.Cu) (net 2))
 (segment (start 150.83 91.47) (end 151.78 92.42) (width 0.25) (layer B.Cu) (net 2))
 (segment (start 149.834998 91.47) (end 150.83 91.47) (width 0.25) (layer B.Cu) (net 2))
 (segment (start 154.139987 93.275002) (end 154.790001 92.624988) (width 0.25) (layer B.Cu) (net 2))
 (segment (start 147.82 89.455002) (end 149.834998 91.47) (width 0.25) (layer B.Cu) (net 2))
 (segment (start 148.632496 91.540319) (end 150.367179 93.275002) (width 0.25) (layer B.Cu) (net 2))
 (segment (start 144.280856 91.540319) (end 148.632496 91.540319) (width 0.25) (layer B.Cu) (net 2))
 (segment (start 147.82 87.36) (end 147.82 89.455002) (width 0.25) (layer B.Cu) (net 2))
 (segment (start 148.583501 85.656499) (end 147.82 86.42) (width 0.25) (layer F.Cu) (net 2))
 (segment (start 147.82 86.42) (end 147.82 87.36) (width 0.25) (layer F.Cu) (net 2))
 (segment (start 148.583501 84.646499) (end 148.583501 85.656499) (width 0.25) (layer F.Cu) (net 2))
 (segment (start 149.383501 83.846499) (end 148.583501 84.646499) (width 0.25) (layer F.Cu) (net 2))
 (segment (start 152.64 84.87) (end 151.616499 83.846499) (width 0.25) (layer F.Cu) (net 2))
 (segment (start 151.616499 83.846499) (end 149.383501 83.846499) (width 0.25) (layer F.Cu) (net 2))
 (segment (start 144.6 91.97) (end 144.280856 91.650856) (width 0.25) (layer F.Cu) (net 2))
 (segment (start 144.280856 91.650856) (end 144.280856 91.540319) (width 0.25) (layer F.Cu) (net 2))
 (segment (start 145.38 91.97) (end 144.6 91.97) (width 0.25) (layer F.Cu) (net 2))
 (segment (start 134.925 92.14) (end 136.173002 92.14) (width 0.25) (layer B.Cu) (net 2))
 (segment (start 143.715171 91.540319) (end 144.280856 91.540319) (width 0.25) (layer B.Cu) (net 2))
 (segment (start 139.049681 91.540319) (end 143.715171 91.540319) (width 0.25) (layer B.Cu) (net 2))
 (segment (start 137.77 92.82) (end 139.049681 91.540319) (width 0.25) (layer B.Cu) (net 2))
 (segment (start 136.853002 92.82) (end 137.77 92.82) (width 0.25) (layer B.Cu) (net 2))
 (segment (start 136.173002 92.14) (end 136.853002 92.82) (width 0.25) (layer B.Cu) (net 2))
 (segment (start 134.925 92.14) (end 133.9 92.14) (width 0.25) (layer B.Cu) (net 2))
 (segment (start 137.21 92.94) (end 136.6 92.33) (width 0.25) (layer F.Cu) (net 2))
 (segment (start 136.6 92.33) (end 136.6 91.14) (width 0.25) (layer F.Cu) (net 2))
 (segment (start 138.29 92.94) (end 137.21 92.94) (width 0.25) (layer F.Cu) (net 2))
 (segment (start 136.6 91.14) (end 137.74 91.14) (width 0.25) (layer F.Cu) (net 2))
 (segment (start 137.74 91.14) (end 138.29 91.69) (width 0.25) (layer F.Cu) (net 2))
 (segment (start 138.29 91.59) (end 138.11 91.77) (width 0.25) (layer F.Cu) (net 2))
 (segment (start 133.9 85.14) (end 133.9 84.39) (width 0.25) (layer B.Cu) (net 2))
 (segment (start 136.62 91.16) (end 136.6 91.14) (width 0.25) (layer F.Cu) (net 2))
 (segment (start 145.05 88.01) (end 145.05 86.71) (width 0.25) (layer F.Cu) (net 2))
 (segment (start 143.75 88.01) (end 145.05 88.01) (width 0.25) (layer F.Cu) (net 2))
 (segment (start 143.75 86.71) (end 143.75 88.01) (width 0.25) (layer F.Cu) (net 2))
 (segment (start 142.45 86.61) (end 143.65 86.61) (width 0.25) (layer F.Cu) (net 2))
 (segment (start 143.65 86.61) (end 143.75 86.71) (width 0.25) (layer F.Cu) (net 2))
 (segment (start 133.9 85.14) (end 135.75 85.14) (width 0.25) (layer B.Cu) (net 2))
 (segment (start 135.75 85.14) (end 136.6 85.99) (width 0.25) (layer B.Cu) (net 2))
 (segment (start 136.6 85.99) (end 136.6 86.14) (width 0.25) (layer B.Cu) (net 2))
 (segment (start 133.9 92.14) (end 133.9 85.14) (width 0.25) (layer B.Cu) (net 2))
 (segment (start 136.6 91.14) (end 136.6 91.29) (width 0.25) (layer B.Cu) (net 2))
 (segment (start 136.6 91.29) (end 135.75 92.14) (width 0.25) (layer B.Cu) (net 2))
 (segment (start 135.75 92.14) (end 134.925 92.14) (width 0.25) (layer B.Cu) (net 2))
 (segment (start 136.6 91.14) (end 136.6 89.94) (width 0.25) (layer F.Cu) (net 2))
 (segment (start 140.356109 86.295008) (end 138.965157 86.295008) (width 0.25) (layer F.Cu) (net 7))
 (segment (start 142.45 87.11) (end 141.171101 87.11) (width 0.25) (layer F.Cu) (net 7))
 (segment (start 138.395174 86.864991) (end 137.995175 87.26499) (width 0.25) (layer F.Cu) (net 7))
 (segment (start 141.171101 87.11) (end 140.356109 86.295008) (width 0.25) (layer F.Cu) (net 7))
 (segment (start 138.965157 86.295008) (end 138.395174 86.864991) (width 0.25) (layer F.Cu) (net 7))
 (segment (start 138.05 89.709998) (end 138.05 87.319815) (width 0.25) (layer B.Cu) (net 7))
 (segment (start 138.05 87.319815) (end 137.995175 87.26499) (width 0.25) (layer B.Cu) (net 7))
 (segment (start 136.6 88.64) (end 137.525 88.64) (width 0.25) (layer F.Cu) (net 7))
 (segment (start 137.525 88.64) (end 138.05 89.165) (width 0.25) (layer F.Cu) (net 7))
 (segment (start 138.05 89.165) (end 138.05 89.709998) (width 0.25) (layer F.Cu) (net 7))
 (segment (start 137.995175 87.365175) (end 137.995175 87.26499) (width 0.25) (layer B.Cu) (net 7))
 (segment (start 138.14 87.51) (end 137.995175 87.365175) (width 0.25) (layer B.Cu) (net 7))
 (segment (start 142.43 87.09) (end 142.45 87.11) (width 0.25) (layer F.Cu) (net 7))
 (segment (start 139.471999 86.724999) (end 140.168001 86.724999) (width 0.25) (layer F.Cu) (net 6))
 (segment (start 141.053002 87.61) (end 141.775 87.61) (width 0.25) (layer F.Cu) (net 6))
 (segment (start 140.168001 86.724999) (end 141.053002 87.61) (width 0.25) (layer F.Cu) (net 6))
 (segment (start 138.606998 87.99) (end 139.054999 87.541999) (width 0.25) (layer F.Cu) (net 6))
 (segment (start 139.054999 87.141999) (end 139.471999 86.724999) (width 0.25) (layer F.Cu) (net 6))
 (segment (start 139.054999 87.541999) (end 139.054999 87.141999) (width 0.25) (layer F.Cu) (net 6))
 (segment (start 141.775 87.61) (end 142.45 87.61) (width 0.25) (layer F.Cu) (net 6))
 (segment (start 136.6 87.99) (end 138.606998 87.99) (width 0.25) (layer F.Cu) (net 6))
 (segment (start 148.79266 86.99) (end 148.392661 86.590001) (width 0.25) (layer B.Cu) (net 3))
 (segment (start 144.279664 86.590001) (end 142.750276 85.060613) (width 0.25) (layer B.Cu) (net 3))
 (segment (start 148.392661 86.590001) (end 144.279664 86.590001) (width 0.25) (layer B.Cu) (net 3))
 (segment (start 142.750276 85.060613) (end 142.350277 84.660614) (width 0.25) (layer B.Cu) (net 3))
 (segment (start 148.79266 86.17734) (end 148.79266 86.88) (width 0.25) (layer F.Cu) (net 3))
 (segment (start 148.79266 86.99) (end 148.79266 89.207658) (width 0.25) (layer F.Cu) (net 3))
 (segment (start 148.79266 86.88) (end 148.79266 86.99) (width 0.25) (layer F.Cu) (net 3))
 (segment (start 144.65 84.735) (end 144.287176 84.372176) (width 0.25) (layer F.Cu) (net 3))
 (segment (start 144.287176 84.372176) (end 143.2044 84.372176) (width 0.25) (layer F.Cu) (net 3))
 (segment (start 144.65 85.41) (end 144.65 84.735) (width 0.25) (layer F.Cu) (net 3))
 (segment (start 143.2044 84.372176) (end 142.915962 84.660614) (width 0.25) (layer F.Cu) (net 3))
 (segment (start 142.915962 84.660614) (end 142.350277 84.660614) (width 0.25) (layer F.Cu) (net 3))
 (segment (start 148.79266 89.207658) (end 149.340003 89.755001) (width 0.25) (layer F.Cu) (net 3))
 (segment (start 152.200001 89.429999) (end 152.95 88.68) (width 0.25) (layer F.Cu) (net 3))
 (segment (start 149.340003 89.755001) (end 149.340003 89.760003) (width 0.25) (layer F.Cu) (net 3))
 (segment (start 149.340003 89.760003) (end 149.63 90.05) (width 0.25) (layer F.Cu) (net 3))
 (segment (start 149.63 90.05) (end 151.58 90.05) (width 0.25) (layer F.Cu) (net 3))
 (segment (start 151.58 90.05) (end 152.200001 89.429999) (width 0.25) (layer F.Cu) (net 3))
 (segment (start 150.1 84.87) (end 152.75 87.52) (width 0.25) (layer F.Cu) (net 3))
 (segment (start 152.75 87.52) (end 152.75 88.68) (width 0.25) (layer F.Cu) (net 3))
 (segment (start 150.1 84.87) (end 148.79266 86.17734) (width 0.25) (layer F.Cu) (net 3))
 (segment (start 145.998682 84.29651) (end 145.58849 84.29651) (width 0.25) (layer F.Cu) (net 4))
 (segment (start 145.15 84.735) (end 145.15 85.41) (width 0.25) (layer F.Cu) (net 4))
 (segment (start 147.56 84.87) (end 146.572172 84.87) (width 0.25) (layer F.Cu) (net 4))
 (segment (start 146.572172 84.87) (end 145.998682 84.29651) (width 0.25) (layer F.Cu) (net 4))
 (segment (start 145.58849 84.29651) (end 145.15 84.735) (width 0.25) (layer F.Cu) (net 4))
 (segment (start 151.05 88.68) (end 149.75141 88.68) (width 0.25) (layer F.Cu) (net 4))
 (segment (start 149.75141 88.68) (end 149.520866 88.910544) (width 0.25) (layer F.Cu) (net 4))
 (segment (start 149.519042 88.912368) (end 149.520866 88.910544) (width 0.25) (layer B.Cu) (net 4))
 (segment (start 149.502368 88.912368) (end 149.519042 88.912368) (width 0.25) (layer B.Cu) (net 4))
 (segment (start 149.52 88.67) (end 149.52 88.909678) (width 0.25) (layer B.Cu) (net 4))
 (segment (start 149.520866 88.344859) (end 149.520866 88.910544) (width 0.25) (layer B.Cu) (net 4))
 (segment (start 148.547828 84.87) (end 149.520866 85.843038) (width 0.25) (layer B.Cu) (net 4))
 (segment (start 149.519999 88.909677) (end 149.520866 88.910544) (width 0.25) (layer F.Cu) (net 4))
 (segment (start 147.56 84.87) (end 148.547828 84.87) (width 0.25) (layer B.Cu) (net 4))
 (segment (start 149.52 88.909678) (end 149.520866 88.910544) (width 0.25) (layer B.Cu) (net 4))
 (segment (start 149.519999 88.670001) (end 149.519999 88.909677) (width 0.25) (layer F.Cu) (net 4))
 (segment (start 149.520866 85.843038) (end 149.520866 88.344859) (width 0.25) (layer B.Cu) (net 4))
 (segment (start 147.114694 90.365306) (end 147.54 89.94) (width 0.25) (layer F.Cu) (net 10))
 (segment (start 144.15 89.31) (end 144.15 89.970002) (width 0.25) (layer F.Cu) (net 10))
 (segment (start 144.545304 90.365306) (end 147.114694 90.365306) (width 0.25) (layer F.Cu) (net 10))
 (segment (start 144.15 89.970002) (end 144.545304 90.365306) (width 0.25) (layer F.Cu) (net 10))
 (via (at 139.35 89.709998) (size 0.8) (drill 0.4) (layers F.Cu B.Cu) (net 1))
 (via (at 140.890135 84.647166) (size 0.8) (drill 0.4) (layers F.Cu B.Cu) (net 1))
 (via (at 150.72 92.55) (size 0.8) (drill 0.4) (layers F.Cu B.Cu) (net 1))
 (via (at 142.111204 92.33099) (size 0.8) (drill 0.4) (layers F.Cu B.Cu) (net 5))
 (via (at 135.93 92.93) (size 0.8) (drill 0.4) (layers F.Cu B.Cu) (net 5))
 (via (at 147.48 93.02) (size 0.8) (drill 0.4) (layers F.Cu B.Cu) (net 5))
 (via (at 139.82 87.45) (size 0.8) (drill 0.4) (layers F.Cu B.Cu) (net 9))
 (via (at 143.834685 92.435279) (size 0.8) (drill 0.4) (layers F.Cu B.Cu) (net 9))
 (via (at 148.645924 92.611244) (size 0.8) (drill 0.4) (layers F.Cu B.Cu) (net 9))
 (via (at 137.38 92.05) (size 0.8) (drill 0.4) (layers F.Cu B.Cu) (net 9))
 (via (at 142.177321 90.325439) (size 0.8) (drill 0.4) (layers F.Cu B.Cu) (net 9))
 (via (at 154.77 91.89) (size 0.8) (drill 0.4) (layers F.Cu B.Cu) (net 2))
 (via (at 147.82 87.36) (size 0.8) (drill 0.4) (layers F.Cu B.Cu) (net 2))
 (via (at 144.280856 91.540319) (size 0.8) (drill 0.4) (layers F.Cu B.Cu) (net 2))
 (via (at 138.05 89.709998) (size 0.8) (drill 0.4) (layers F.Cu B.Cu) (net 7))
 (via (at 137.995175 87.26499) (size 0.8) (drill 0.4) (layers F.Cu B.Cu) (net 7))
 (via (at 148.79266 86.99) (size 0.8) (drill 0.4) (layers F.Cu B.Cu) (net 3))
 (via (at 142.350277 84.660614) (size 0.8) (drill 0.4) (layers F.Cu B.Cu) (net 3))
 (via (at 149.520866 88.910544) (size 0.8) (drill 0.4) (layers F.Cu B.Cu) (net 4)))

